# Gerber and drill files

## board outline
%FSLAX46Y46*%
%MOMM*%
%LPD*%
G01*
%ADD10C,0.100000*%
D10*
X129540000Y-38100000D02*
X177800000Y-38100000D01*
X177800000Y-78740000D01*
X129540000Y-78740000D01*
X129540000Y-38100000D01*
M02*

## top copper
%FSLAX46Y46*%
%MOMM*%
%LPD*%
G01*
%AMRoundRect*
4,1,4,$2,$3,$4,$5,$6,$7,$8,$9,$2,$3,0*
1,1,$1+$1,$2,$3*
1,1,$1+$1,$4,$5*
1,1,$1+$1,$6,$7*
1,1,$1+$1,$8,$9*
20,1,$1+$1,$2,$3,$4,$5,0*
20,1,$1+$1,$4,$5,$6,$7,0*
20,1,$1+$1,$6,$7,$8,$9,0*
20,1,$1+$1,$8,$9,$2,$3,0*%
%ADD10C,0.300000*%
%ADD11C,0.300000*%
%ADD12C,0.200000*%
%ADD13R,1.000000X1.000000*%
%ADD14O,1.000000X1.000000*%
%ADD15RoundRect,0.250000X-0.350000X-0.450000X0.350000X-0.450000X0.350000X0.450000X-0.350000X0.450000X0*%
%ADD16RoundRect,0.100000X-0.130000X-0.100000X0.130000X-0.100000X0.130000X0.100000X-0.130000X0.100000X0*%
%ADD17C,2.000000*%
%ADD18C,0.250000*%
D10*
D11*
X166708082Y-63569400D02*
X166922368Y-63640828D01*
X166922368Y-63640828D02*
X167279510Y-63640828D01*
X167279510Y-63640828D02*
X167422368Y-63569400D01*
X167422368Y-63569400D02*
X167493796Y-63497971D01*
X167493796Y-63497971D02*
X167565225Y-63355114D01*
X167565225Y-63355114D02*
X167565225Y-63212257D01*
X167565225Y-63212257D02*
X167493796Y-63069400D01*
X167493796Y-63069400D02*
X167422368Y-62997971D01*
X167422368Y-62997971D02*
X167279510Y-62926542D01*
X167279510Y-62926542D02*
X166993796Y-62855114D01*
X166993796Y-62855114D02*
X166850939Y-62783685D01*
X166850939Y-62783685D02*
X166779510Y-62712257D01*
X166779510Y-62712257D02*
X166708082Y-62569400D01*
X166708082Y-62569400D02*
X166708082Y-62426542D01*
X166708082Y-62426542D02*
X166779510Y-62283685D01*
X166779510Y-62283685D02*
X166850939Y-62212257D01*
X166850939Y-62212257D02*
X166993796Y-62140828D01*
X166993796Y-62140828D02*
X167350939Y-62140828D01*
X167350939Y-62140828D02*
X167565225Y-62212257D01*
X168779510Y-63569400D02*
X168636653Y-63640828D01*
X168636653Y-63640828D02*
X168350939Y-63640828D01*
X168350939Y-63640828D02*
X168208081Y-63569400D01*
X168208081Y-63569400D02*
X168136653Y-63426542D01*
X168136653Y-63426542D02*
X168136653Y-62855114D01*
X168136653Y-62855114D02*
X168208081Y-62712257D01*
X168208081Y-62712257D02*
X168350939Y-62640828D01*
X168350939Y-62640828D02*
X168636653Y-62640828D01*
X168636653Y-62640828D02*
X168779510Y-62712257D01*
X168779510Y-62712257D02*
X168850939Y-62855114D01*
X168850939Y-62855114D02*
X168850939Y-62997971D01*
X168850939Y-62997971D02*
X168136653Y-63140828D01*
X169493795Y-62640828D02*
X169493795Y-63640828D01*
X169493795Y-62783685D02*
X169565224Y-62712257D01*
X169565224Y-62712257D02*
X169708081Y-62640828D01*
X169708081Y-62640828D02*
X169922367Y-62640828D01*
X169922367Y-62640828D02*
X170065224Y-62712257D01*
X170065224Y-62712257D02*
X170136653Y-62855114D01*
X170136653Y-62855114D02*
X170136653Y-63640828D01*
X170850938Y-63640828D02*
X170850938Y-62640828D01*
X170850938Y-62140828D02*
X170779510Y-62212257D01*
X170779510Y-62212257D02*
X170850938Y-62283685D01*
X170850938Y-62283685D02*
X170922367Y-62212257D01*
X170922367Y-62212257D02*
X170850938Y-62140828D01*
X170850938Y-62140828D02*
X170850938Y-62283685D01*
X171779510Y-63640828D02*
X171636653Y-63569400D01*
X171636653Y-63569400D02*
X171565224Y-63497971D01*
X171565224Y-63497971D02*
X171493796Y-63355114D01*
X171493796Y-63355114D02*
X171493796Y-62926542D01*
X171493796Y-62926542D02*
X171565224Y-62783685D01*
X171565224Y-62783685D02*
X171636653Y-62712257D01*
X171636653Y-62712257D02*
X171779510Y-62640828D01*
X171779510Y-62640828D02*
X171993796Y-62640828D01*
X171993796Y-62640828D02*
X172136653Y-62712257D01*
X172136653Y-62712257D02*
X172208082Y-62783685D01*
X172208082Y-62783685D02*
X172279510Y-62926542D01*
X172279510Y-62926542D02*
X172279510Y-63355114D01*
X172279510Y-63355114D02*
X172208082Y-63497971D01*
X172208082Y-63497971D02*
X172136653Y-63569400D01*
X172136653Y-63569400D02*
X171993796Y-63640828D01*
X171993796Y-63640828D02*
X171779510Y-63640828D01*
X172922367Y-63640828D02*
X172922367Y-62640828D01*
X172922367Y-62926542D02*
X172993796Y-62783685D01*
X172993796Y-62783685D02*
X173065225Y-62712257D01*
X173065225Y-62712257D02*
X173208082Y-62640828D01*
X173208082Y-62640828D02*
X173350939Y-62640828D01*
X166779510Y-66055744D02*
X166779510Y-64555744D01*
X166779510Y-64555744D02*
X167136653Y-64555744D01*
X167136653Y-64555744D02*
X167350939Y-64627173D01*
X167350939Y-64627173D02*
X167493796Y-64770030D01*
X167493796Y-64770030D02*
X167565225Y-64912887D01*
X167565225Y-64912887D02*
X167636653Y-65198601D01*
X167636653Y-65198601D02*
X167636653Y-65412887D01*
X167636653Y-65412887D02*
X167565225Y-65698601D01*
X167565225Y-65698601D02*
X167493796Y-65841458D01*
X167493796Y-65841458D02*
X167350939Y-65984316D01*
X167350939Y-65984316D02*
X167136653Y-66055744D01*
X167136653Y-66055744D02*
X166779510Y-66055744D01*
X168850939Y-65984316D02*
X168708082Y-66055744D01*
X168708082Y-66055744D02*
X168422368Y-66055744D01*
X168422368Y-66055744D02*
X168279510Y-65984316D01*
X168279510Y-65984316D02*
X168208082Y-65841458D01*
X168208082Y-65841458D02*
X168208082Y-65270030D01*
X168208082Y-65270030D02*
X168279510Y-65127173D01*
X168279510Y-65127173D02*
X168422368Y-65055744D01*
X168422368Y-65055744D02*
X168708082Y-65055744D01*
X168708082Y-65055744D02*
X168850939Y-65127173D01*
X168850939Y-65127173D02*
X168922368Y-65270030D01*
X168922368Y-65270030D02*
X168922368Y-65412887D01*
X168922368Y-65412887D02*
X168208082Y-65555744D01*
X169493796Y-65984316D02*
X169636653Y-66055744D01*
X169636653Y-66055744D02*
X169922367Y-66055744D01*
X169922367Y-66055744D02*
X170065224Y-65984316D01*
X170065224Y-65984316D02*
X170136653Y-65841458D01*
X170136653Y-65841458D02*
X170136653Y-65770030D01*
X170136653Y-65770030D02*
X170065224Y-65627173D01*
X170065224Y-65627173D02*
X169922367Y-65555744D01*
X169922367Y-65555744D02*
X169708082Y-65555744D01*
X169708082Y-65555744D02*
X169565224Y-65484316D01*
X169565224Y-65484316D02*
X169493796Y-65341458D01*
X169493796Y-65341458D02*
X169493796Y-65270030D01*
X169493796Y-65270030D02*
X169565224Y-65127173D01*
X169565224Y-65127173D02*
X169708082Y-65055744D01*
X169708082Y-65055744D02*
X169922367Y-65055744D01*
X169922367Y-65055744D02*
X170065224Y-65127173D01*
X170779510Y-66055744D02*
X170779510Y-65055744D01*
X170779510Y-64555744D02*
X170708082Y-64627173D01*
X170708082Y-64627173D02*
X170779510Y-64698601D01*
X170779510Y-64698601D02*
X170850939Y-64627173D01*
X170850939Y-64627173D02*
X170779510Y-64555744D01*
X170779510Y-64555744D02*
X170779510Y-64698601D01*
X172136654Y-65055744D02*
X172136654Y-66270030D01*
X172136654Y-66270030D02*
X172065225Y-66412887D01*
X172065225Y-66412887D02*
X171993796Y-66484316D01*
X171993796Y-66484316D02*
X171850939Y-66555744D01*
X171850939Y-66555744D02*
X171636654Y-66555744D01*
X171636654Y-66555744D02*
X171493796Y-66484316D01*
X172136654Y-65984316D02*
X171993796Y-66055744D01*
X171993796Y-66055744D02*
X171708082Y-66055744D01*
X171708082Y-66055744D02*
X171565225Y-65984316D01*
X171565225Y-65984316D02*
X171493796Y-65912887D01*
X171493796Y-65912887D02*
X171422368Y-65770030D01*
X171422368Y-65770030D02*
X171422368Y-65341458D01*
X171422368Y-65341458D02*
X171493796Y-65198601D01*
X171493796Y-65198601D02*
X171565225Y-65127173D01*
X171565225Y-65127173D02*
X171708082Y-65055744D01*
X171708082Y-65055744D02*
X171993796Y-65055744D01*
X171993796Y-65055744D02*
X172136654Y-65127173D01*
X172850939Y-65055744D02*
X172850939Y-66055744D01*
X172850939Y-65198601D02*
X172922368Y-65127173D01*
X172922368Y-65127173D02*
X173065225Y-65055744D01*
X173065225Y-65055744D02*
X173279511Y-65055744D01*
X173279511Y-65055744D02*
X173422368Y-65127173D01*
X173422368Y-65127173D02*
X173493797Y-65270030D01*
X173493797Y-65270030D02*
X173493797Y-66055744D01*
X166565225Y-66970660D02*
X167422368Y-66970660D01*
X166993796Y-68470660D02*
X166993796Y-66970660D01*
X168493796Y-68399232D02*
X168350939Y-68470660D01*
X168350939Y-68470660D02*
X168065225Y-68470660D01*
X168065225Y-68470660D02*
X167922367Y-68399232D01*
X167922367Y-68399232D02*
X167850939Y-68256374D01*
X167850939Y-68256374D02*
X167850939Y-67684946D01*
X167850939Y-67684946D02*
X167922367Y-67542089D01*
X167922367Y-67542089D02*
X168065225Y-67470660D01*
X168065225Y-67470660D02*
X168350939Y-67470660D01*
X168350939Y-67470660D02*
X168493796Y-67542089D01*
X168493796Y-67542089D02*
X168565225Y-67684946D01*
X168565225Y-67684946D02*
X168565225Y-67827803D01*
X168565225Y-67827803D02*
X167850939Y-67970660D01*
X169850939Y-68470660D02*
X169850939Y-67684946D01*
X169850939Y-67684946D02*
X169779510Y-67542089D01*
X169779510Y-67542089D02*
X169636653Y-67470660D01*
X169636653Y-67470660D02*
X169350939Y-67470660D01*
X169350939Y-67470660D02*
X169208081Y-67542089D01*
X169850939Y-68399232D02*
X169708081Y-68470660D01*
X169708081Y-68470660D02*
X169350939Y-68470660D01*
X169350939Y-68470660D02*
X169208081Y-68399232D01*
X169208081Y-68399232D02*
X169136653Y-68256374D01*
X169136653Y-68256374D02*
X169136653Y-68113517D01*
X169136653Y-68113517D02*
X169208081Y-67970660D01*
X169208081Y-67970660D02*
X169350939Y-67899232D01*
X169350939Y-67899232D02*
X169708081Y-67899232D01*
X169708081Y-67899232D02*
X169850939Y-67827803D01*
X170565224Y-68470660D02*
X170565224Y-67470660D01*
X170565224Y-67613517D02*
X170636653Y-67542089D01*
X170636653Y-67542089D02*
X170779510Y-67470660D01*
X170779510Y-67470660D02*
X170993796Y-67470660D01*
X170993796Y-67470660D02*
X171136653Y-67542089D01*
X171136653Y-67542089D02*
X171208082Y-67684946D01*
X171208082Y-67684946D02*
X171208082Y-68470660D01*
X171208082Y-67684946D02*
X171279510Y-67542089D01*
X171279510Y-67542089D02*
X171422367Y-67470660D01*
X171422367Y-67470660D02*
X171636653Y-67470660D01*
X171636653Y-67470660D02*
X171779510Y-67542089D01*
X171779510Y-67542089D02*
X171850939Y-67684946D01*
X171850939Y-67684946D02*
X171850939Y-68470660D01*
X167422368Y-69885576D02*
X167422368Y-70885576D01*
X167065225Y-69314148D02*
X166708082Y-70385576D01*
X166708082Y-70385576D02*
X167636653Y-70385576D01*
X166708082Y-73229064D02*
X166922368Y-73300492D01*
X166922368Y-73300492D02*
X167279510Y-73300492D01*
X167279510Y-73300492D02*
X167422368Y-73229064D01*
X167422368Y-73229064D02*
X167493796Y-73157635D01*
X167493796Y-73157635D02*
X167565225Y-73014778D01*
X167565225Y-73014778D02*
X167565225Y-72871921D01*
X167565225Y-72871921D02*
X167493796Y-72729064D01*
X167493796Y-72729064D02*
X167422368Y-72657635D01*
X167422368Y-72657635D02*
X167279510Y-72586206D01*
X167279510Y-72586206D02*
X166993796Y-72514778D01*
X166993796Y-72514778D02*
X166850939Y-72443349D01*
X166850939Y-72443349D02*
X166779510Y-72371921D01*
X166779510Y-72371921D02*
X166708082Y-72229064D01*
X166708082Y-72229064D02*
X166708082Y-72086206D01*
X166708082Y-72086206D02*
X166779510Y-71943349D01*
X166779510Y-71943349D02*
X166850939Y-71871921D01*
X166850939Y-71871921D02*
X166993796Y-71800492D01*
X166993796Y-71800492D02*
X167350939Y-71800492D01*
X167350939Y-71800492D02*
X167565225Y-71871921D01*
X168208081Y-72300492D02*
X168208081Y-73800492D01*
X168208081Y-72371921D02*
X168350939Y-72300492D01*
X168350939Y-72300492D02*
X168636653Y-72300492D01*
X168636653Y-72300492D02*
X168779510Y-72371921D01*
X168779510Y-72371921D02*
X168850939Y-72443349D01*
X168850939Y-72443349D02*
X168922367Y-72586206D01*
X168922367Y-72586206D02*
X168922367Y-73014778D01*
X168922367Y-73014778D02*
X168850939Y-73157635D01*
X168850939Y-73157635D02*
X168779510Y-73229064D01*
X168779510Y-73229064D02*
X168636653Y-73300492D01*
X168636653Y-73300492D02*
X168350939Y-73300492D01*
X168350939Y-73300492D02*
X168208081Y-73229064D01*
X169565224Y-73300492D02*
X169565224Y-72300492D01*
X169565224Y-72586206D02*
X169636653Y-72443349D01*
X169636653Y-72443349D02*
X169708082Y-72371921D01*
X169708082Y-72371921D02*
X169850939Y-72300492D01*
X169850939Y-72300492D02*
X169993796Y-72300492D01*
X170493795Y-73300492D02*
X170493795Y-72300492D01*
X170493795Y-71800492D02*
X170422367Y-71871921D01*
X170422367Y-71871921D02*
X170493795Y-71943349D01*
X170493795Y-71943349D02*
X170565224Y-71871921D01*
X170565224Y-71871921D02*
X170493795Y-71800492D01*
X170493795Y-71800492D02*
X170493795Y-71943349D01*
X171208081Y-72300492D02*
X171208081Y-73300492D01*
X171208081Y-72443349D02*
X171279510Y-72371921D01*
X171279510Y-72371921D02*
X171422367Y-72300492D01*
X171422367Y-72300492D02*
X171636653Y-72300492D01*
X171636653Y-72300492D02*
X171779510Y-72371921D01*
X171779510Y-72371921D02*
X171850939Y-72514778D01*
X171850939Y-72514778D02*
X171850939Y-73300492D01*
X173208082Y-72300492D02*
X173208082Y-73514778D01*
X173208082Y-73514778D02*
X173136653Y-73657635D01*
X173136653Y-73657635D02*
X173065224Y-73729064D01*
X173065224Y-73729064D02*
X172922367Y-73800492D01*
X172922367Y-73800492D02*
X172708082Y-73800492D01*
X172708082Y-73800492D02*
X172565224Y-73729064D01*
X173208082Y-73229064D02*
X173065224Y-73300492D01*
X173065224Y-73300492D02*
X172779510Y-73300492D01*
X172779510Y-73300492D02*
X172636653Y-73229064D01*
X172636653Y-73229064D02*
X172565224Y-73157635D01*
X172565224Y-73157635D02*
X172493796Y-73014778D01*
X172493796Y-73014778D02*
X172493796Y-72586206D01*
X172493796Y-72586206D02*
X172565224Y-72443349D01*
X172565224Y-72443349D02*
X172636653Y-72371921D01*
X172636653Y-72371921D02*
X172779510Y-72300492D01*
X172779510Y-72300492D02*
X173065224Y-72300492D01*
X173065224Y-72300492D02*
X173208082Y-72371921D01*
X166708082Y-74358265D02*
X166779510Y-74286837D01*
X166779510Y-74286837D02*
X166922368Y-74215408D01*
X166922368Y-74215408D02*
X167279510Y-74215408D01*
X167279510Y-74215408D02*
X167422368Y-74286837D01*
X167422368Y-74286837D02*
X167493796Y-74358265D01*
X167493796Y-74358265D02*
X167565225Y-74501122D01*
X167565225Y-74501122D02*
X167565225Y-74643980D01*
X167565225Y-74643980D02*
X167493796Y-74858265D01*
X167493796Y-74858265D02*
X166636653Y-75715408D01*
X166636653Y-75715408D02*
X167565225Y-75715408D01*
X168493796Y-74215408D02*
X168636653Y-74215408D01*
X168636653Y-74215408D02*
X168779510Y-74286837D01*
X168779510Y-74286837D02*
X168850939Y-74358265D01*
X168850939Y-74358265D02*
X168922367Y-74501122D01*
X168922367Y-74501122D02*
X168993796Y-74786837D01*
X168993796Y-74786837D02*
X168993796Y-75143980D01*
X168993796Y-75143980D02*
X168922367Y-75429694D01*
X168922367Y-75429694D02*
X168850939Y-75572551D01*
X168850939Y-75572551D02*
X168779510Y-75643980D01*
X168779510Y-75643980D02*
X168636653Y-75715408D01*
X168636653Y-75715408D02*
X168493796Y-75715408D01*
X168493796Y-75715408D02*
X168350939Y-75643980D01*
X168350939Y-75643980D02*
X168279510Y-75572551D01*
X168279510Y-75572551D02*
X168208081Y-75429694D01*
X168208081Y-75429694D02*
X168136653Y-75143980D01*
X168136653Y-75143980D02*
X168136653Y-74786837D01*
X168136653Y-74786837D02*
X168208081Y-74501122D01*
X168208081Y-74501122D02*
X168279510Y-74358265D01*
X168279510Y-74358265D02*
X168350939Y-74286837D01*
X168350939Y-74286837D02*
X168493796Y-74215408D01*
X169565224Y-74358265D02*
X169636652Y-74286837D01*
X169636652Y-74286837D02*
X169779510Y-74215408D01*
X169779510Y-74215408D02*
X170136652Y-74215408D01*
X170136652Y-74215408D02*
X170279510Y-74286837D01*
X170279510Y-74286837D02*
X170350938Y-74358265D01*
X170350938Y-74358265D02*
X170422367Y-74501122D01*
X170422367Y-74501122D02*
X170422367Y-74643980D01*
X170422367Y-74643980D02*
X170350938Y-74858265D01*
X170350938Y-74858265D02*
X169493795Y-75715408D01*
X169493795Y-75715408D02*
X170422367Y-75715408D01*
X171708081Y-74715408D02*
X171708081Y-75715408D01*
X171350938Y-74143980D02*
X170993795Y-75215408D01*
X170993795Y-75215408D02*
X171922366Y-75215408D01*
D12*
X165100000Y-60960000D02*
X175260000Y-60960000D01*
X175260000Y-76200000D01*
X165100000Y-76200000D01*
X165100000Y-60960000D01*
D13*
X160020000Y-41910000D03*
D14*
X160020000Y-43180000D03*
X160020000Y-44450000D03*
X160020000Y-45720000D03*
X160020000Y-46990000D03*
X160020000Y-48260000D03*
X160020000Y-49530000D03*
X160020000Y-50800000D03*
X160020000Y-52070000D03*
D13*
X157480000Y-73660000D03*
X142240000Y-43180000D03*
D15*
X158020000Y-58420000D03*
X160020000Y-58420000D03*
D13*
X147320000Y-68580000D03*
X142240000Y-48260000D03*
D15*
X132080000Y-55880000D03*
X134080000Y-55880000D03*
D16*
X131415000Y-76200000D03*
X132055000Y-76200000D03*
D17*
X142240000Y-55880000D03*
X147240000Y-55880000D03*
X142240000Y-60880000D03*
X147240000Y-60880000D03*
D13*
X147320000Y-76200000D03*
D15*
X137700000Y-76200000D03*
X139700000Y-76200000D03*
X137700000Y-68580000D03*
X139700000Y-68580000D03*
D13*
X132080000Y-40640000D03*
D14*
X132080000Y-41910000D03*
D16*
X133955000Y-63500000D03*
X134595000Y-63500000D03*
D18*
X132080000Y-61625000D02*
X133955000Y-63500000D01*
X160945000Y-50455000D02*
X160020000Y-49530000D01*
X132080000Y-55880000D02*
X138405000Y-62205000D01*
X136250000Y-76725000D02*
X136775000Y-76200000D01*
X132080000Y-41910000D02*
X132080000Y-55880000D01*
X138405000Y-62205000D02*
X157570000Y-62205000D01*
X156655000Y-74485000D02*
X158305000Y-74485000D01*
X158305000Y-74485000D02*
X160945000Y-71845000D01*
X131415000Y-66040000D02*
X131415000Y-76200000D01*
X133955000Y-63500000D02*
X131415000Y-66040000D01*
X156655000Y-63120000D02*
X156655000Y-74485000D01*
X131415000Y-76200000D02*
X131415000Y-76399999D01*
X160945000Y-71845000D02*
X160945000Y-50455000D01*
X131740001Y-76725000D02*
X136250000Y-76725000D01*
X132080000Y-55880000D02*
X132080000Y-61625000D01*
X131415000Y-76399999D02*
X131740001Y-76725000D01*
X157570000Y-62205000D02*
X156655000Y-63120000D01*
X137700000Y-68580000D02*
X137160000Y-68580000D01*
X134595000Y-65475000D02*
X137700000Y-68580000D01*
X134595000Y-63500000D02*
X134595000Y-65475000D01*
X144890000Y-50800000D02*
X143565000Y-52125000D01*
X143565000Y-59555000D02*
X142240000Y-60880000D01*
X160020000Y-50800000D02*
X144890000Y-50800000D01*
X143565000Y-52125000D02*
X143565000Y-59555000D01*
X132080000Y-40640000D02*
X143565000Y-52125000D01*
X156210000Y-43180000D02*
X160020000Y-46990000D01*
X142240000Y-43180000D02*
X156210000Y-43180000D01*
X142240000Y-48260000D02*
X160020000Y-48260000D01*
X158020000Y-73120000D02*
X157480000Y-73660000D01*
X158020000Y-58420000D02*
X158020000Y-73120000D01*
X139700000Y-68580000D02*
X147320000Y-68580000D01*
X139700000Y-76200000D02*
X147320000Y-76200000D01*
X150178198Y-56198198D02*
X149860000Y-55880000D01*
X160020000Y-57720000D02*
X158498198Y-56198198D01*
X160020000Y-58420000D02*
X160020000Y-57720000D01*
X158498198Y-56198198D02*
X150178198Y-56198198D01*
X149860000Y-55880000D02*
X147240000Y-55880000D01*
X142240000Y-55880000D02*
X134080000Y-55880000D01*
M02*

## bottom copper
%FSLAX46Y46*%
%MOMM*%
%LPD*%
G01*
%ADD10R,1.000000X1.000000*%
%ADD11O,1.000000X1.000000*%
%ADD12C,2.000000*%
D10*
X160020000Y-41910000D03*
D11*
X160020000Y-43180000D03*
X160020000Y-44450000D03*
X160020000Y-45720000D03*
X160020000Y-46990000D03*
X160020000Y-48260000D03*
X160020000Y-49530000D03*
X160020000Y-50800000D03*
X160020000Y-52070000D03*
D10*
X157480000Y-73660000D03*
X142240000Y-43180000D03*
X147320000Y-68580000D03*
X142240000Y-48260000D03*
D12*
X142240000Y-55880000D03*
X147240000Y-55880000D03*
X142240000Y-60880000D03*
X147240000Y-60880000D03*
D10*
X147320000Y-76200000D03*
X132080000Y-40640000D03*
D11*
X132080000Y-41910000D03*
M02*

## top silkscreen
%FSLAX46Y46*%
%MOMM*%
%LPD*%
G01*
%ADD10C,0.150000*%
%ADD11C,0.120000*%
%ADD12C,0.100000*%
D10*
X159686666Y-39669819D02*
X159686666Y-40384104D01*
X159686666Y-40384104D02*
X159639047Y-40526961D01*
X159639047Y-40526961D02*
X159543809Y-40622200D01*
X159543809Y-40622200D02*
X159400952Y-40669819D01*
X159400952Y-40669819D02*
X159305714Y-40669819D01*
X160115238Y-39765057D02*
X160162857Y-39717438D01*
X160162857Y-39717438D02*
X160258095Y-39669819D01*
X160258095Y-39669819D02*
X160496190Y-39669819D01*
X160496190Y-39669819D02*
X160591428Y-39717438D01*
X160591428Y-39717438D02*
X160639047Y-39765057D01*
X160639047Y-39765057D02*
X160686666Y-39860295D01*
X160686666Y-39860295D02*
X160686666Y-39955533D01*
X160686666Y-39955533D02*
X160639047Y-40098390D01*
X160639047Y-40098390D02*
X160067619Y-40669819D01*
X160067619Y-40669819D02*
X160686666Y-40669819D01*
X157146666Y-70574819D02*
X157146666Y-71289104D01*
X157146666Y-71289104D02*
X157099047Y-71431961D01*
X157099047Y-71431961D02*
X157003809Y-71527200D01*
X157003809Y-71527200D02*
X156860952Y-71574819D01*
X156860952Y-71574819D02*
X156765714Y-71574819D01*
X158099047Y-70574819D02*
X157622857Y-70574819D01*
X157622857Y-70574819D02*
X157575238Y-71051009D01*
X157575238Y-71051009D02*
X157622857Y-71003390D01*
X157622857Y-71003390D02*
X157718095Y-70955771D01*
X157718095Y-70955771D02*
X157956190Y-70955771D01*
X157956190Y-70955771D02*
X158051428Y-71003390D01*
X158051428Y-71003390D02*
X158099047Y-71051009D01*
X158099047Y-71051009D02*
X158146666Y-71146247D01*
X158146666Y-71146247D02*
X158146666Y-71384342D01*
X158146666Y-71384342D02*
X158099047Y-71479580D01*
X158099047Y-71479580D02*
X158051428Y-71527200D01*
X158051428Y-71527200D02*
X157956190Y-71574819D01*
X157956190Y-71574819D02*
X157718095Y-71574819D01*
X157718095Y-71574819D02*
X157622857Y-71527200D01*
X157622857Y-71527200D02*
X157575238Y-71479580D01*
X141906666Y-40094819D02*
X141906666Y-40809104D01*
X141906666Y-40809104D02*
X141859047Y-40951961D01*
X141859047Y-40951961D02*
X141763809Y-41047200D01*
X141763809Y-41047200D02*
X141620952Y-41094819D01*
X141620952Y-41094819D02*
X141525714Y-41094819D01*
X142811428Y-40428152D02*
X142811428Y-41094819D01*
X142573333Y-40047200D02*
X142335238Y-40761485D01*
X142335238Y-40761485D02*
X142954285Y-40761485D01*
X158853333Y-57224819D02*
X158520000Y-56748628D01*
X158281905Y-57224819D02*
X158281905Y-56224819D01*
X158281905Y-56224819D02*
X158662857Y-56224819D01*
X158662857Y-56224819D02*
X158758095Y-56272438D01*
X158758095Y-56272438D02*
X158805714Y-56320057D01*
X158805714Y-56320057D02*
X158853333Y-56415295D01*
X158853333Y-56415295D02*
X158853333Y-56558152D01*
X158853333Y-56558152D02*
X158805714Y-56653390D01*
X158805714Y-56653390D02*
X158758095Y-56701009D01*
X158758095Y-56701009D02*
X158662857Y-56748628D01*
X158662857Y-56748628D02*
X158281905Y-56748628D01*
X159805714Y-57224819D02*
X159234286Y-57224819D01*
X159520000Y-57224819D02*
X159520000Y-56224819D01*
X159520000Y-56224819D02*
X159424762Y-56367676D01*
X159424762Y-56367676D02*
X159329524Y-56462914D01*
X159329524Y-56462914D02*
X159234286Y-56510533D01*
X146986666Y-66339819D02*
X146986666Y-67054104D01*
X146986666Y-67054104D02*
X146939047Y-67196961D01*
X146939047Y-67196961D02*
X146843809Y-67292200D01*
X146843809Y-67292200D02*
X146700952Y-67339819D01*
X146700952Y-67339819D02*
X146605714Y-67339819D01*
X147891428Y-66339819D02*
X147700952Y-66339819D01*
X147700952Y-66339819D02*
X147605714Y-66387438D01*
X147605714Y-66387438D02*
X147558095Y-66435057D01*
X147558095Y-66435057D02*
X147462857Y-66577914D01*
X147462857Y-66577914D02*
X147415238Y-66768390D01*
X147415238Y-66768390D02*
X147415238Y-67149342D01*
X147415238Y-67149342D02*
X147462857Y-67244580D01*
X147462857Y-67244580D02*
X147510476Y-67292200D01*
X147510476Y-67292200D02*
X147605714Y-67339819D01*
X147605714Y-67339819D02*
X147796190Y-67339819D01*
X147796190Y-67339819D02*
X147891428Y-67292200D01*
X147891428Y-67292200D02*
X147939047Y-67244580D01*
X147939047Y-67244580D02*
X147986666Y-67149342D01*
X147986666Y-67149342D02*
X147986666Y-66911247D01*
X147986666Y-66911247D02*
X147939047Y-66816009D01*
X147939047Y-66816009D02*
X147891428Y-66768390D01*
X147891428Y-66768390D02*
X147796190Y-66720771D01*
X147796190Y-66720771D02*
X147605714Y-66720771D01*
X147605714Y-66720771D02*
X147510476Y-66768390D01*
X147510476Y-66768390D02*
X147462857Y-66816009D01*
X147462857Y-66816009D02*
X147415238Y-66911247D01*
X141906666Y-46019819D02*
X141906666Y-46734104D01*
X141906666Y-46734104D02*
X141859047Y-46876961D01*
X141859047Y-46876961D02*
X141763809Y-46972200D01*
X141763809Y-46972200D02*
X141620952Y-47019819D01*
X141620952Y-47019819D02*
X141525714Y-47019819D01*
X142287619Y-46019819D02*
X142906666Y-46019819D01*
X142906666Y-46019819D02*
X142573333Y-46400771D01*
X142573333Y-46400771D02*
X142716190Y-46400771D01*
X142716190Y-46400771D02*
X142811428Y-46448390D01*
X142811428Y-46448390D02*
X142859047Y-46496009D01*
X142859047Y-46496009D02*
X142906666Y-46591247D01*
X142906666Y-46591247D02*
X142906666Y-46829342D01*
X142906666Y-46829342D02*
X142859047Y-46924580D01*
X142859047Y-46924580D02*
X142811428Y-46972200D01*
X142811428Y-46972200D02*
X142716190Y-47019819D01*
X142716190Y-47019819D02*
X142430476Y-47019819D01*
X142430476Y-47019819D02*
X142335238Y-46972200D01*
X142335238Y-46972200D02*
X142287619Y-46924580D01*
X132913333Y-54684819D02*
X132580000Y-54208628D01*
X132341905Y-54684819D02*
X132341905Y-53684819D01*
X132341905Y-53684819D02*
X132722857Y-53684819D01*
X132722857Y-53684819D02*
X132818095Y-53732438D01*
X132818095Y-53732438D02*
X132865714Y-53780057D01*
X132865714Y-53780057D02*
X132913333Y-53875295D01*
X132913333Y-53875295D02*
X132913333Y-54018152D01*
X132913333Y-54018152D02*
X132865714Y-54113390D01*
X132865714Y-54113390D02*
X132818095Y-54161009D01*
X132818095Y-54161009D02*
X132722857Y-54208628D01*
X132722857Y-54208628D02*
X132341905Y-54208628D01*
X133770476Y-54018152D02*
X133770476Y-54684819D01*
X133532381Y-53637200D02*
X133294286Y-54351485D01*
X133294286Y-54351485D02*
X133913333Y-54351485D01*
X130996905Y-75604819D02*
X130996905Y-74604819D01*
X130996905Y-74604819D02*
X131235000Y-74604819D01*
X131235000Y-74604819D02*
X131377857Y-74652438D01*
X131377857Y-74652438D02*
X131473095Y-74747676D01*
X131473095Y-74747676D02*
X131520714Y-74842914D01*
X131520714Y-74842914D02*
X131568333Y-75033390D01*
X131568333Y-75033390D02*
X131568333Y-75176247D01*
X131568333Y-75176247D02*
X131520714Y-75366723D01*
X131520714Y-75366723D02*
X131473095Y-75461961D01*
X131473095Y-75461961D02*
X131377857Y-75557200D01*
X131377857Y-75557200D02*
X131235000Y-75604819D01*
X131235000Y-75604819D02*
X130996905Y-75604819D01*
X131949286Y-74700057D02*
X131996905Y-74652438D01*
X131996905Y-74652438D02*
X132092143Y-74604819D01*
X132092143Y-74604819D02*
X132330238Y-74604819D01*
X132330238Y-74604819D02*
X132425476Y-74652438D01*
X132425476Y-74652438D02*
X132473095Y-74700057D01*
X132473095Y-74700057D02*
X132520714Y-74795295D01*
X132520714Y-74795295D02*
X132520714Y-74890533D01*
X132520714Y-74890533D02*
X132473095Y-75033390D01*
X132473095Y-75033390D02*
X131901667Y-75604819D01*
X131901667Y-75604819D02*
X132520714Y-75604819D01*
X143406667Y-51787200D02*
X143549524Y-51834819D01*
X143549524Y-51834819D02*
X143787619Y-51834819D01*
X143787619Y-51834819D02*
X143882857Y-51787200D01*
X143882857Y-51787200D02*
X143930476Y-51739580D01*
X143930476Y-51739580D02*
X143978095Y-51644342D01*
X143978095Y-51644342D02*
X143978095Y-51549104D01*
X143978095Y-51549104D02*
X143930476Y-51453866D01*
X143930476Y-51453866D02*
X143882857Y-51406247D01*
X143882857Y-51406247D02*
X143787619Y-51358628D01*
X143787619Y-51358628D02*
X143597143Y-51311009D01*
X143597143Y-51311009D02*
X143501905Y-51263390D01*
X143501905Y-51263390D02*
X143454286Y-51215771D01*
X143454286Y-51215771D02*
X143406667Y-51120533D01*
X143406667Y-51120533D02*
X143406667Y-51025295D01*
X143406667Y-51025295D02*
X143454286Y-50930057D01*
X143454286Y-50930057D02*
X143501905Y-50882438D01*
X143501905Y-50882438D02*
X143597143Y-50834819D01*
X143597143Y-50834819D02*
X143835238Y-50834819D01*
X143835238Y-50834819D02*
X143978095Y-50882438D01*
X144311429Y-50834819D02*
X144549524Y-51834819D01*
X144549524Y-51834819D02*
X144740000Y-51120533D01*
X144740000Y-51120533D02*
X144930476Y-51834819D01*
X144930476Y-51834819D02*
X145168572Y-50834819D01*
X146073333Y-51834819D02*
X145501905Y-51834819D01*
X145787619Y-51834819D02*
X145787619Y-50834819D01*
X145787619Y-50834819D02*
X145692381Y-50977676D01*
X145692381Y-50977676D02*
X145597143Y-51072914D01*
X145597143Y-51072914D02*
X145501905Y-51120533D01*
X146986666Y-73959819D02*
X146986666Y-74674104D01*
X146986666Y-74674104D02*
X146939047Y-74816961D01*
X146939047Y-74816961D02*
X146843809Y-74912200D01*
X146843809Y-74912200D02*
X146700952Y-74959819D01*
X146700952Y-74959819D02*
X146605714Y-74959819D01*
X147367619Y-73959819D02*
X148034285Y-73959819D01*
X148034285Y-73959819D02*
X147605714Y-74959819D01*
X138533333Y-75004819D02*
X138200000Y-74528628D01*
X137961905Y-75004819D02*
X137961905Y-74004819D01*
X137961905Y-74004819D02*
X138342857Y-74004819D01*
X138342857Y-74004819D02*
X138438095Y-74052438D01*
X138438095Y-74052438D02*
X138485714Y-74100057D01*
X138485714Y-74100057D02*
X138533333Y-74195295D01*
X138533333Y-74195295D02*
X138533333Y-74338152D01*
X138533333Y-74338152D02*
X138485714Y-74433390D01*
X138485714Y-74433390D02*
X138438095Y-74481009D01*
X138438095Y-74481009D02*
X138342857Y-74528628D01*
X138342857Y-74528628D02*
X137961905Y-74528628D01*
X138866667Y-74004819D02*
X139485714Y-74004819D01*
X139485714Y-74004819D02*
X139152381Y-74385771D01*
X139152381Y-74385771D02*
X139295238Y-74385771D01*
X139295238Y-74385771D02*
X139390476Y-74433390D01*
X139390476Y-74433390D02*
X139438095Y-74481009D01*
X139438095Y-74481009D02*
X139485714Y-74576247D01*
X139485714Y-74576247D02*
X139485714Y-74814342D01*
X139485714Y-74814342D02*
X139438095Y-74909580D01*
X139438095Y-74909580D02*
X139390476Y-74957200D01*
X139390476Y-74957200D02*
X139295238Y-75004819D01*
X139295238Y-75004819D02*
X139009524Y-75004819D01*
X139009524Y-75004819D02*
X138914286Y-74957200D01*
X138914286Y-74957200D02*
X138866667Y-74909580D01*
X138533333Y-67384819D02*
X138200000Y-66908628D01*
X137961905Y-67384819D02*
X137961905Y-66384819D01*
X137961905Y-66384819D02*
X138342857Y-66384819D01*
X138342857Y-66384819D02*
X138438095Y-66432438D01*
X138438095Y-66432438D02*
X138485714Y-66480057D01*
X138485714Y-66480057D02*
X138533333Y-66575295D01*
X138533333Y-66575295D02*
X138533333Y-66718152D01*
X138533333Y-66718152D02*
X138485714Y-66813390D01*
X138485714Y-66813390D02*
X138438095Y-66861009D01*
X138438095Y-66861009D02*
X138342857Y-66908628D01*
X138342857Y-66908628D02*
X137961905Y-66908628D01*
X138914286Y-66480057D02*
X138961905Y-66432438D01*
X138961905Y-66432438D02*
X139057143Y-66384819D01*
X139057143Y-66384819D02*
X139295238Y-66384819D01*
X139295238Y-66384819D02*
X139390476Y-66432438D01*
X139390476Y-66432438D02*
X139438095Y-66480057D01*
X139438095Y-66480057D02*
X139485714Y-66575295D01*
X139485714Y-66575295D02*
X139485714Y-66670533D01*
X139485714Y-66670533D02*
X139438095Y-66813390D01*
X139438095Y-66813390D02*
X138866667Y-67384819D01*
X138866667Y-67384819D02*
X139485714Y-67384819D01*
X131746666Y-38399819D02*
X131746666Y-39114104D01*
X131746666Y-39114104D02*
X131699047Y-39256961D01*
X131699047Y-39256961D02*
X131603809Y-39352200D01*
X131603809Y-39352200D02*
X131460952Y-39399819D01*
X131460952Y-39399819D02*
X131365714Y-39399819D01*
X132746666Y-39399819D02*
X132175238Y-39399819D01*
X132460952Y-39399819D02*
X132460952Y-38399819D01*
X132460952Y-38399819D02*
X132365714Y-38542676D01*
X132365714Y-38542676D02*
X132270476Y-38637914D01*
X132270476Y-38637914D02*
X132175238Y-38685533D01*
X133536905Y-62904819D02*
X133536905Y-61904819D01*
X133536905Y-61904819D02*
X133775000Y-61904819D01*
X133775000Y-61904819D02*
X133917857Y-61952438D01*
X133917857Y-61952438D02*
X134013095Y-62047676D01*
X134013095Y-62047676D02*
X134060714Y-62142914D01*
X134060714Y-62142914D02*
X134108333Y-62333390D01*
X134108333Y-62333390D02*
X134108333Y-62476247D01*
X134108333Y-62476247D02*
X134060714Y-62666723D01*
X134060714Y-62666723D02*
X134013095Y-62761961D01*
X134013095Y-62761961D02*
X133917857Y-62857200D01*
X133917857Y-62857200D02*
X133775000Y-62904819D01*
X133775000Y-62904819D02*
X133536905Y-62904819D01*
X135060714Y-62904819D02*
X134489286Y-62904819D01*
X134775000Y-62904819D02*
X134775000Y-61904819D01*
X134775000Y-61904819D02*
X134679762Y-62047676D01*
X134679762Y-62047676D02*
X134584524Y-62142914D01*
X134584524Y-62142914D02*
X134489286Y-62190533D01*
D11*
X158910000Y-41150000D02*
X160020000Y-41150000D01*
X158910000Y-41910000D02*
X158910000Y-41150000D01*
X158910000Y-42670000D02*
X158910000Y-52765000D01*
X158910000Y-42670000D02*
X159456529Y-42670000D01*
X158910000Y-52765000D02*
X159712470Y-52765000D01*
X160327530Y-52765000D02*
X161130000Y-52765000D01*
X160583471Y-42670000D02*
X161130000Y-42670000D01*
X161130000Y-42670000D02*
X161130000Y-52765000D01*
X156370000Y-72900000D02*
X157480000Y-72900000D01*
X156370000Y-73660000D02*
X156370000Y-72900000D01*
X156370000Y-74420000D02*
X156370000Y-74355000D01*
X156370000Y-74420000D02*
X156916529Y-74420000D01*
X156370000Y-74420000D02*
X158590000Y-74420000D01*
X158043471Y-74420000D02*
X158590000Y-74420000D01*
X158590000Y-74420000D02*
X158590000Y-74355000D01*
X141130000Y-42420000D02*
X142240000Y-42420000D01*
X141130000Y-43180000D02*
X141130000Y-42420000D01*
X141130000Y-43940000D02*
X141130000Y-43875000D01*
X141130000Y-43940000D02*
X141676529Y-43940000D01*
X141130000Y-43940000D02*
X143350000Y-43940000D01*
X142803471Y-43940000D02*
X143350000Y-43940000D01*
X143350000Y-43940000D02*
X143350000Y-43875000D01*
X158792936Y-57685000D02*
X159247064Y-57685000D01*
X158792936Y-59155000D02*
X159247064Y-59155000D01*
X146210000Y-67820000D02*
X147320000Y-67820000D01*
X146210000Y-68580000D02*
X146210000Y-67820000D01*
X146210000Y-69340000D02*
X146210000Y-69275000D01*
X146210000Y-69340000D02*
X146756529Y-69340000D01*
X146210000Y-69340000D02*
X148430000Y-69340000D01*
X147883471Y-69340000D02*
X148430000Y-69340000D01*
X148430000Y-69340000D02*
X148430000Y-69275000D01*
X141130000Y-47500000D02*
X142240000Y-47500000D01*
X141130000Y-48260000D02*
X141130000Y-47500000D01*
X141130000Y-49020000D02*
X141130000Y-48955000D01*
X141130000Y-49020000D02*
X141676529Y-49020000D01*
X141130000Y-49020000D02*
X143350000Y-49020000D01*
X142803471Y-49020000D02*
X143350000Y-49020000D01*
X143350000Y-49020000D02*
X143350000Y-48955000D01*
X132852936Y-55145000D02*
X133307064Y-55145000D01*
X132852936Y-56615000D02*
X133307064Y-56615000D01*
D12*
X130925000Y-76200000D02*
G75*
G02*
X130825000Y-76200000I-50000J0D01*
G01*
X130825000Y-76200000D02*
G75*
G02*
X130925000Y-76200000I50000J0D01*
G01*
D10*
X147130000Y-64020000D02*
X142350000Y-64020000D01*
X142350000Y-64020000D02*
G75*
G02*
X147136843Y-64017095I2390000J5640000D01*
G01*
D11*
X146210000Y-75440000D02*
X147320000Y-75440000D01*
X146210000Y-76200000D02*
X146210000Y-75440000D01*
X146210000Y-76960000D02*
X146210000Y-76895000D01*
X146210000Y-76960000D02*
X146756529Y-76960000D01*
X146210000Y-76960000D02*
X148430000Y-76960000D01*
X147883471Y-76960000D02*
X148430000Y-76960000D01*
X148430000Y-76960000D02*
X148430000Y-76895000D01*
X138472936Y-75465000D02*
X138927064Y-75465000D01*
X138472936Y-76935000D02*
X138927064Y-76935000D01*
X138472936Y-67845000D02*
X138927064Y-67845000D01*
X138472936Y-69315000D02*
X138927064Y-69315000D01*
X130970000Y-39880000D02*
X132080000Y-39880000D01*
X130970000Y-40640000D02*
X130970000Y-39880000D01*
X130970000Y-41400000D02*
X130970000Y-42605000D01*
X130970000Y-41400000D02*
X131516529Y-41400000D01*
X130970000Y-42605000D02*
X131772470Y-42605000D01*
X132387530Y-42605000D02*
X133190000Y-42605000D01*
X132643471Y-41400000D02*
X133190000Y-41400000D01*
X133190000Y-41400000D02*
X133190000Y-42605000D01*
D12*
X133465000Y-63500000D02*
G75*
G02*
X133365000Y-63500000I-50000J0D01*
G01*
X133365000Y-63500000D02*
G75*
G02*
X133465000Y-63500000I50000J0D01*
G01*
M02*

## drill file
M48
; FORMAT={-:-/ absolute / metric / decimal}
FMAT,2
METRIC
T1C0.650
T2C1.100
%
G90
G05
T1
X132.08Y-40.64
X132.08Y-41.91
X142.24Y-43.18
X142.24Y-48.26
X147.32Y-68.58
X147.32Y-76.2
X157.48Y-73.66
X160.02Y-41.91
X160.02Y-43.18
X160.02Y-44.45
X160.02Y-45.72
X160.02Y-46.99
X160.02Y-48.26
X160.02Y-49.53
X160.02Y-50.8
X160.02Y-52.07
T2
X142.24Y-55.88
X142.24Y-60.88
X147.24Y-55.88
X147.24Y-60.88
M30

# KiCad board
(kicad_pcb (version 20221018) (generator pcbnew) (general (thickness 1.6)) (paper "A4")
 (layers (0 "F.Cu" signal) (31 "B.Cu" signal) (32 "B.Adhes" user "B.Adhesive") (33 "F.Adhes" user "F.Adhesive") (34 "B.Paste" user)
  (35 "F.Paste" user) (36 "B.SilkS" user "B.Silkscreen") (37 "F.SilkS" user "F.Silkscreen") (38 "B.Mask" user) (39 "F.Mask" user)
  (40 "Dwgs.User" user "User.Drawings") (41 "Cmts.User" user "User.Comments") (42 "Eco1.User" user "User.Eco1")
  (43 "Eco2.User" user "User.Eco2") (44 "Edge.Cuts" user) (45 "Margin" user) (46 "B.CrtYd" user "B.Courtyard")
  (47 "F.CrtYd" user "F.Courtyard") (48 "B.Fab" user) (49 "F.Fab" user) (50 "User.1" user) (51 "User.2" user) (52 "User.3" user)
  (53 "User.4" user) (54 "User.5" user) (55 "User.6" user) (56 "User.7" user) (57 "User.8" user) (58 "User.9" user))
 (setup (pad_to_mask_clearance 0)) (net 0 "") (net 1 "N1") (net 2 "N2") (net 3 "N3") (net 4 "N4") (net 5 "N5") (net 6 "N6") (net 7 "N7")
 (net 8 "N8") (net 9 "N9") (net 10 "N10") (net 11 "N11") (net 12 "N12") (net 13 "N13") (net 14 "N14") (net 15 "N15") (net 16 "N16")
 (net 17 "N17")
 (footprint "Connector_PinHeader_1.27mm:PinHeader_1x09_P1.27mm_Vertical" (layer "F.Cu") (at 160.02 41.91)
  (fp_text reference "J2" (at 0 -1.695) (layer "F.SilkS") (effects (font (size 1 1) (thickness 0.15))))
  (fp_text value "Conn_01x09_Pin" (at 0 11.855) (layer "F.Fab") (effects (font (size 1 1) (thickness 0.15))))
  (fp_line (start -1.11 -0.76) (end 0 -0.76) (stroke (width 0.12) (type solid)) (layer "F.SilkS"))
  (fp_line (start -1.11 0) (end -1.11 -0.76) (stroke (width 0.12) (type solid)) (layer "F.SilkS"))
  (fp_line (start -1.11 0.76) (end -1.11 10.855) (stroke (width 0.12) (type solid)) (layer "F.SilkS"))
  (fp_line (start -1.11 0.76) (end -0.563471 0.76) (stroke (width 0.12) (type solid)) (layer "F.SilkS"))
  (fp_line (start -1.11 10.855) (end -0.30753 10.855) (stroke (width 0.12) (type solid)) (layer "F.SilkS"))
  (fp_line (start 0.30753 10.855) (end 1.11 10.855) (stroke (width 0.12) (type solid)) (layer "F.SilkS"))
  (fp_line (start 0.563471 0.76) (end 1.11 0.76) (stroke (width 0.12) (type solid)) (layer "F.SilkS"))
  (fp_line (start 1.11 0.76) (end 1.11 10.855) (stroke (width 0.12) (type solid)) (layer "F.SilkS"))
  (pad "1" thru_hole rect (at 0 0) (size 1 1) (drill 0.65) (layers "*.Cu" "*.Mask") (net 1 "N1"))
  (pad "2" thru_hole oval (at 0 1.27) (size 1 1) (drill 0.65) (layers "*.Cu" "*.Mask") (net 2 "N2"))
  (pad "3" thru_hole oval (at 0 2.54) (size 1 1) (drill 0.65) (layers "*.Cu" "*.Mask") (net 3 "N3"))
  (pad "4" thru_hole oval (at 0 3.81) (size 1 1) (drill 0.65) (layers "*.Cu" "*.Mask") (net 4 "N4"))
  (pad "5" thru_hole oval (at 0 5.08) (size 1 1) (drill 0.65) (layers "*.Cu" "*.Mask") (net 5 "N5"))
  (pad "6" thru_hole oval (at 0 6.35) (size 1 1) (drill 0.65) (layers "*.Cu" "*.Mask") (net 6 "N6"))
  (pad "7" thru_hole oval (at 0 7.62) (size 1 1) (drill 0.65) (layers "*.Cu" "*.Mask") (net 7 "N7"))
  (pad "8" thru_hole oval (at 0 8.89) (size 1 1) (drill 0.65) (layers "*.Cu" "*.Mask") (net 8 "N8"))
  (pad "9" thru_hole oval (at 0 10.16) (size 1 1) (drill 0.65) (layers "*.Cu" "*.Mask") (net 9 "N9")))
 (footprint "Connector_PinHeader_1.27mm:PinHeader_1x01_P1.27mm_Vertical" (layer "F.Cu") (at 157.48 73.66)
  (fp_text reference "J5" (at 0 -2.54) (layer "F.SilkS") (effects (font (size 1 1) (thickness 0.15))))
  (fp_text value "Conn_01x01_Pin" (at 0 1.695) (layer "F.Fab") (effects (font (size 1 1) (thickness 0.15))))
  (fp_line (start -1.11 -0.76) (end 0 -0.76) (stroke (width 0.12) (type solid)) (layer "F.SilkS"))
  (fp_line (start -1.11 0) (end -1.11 -0.76) (stroke (width 0.12) (type solid)) (layer "F.SilkS"))
  (fp_line (start -1.11 0.76) (end -1.11 0.695) (stroke (width 0.12) (type solid)) (layer "F.SilkS"))
  (fp_line (start -1.11 0.76) (end -0.563471 0.76) (stroke (width 0.12) (type solid)) (layer "F.SilkS"))
  (fp_line (start -1.11 0.76) (end 1.11 0.76) (stroke (width 0.12) (type solid)) (layer "F.SilkS"))
  (fp_line (start 0.563471 0.76) (end 1.11 0.76) (stroke (width 0.12) (type solid)) (layer "F.SilkS"))
  (fp_line (start 1.11 0.76) (end 1.11 0.695) (stroke (width 0.12) (type solid)) (layer "F.SilkS"))
  (pad "1" thru_hole rect (at 0 0) (size 1 1) (drill 0.65) (layers "*.Cu" "*.Mask") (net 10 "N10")))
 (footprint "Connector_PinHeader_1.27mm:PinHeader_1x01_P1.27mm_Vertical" (layer "F.Cu") (at 142.24 43.18)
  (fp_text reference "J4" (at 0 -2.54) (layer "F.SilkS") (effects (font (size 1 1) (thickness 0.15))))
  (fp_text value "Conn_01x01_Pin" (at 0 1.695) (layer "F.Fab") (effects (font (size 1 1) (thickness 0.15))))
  (fp_line (start -1.11 -0.76) (end 0 -0.76) (stroke (width 0.12) (type solid)) (layer "F.SilkS"))
  (fp_line (start -1.11 0) (end -1.11 -0.76) (stroke (width 0.12) (type solid)) (layer "F.SilkS"))
  (fp_line (start -1.11 0.76) (end -1.11 0.695) (stroke (width 0.12) (type solid)) (layer "F.SilkS"))
  (fp_line (start -1.11 0.76) (end -0.563471 0.76) (stroke (width 0.12) (type solid)) (layer "F.SilkS"))
  (fp_line (start -1.11 0.76) (end 1.11 0.76) (stroke (width 0.12) (type solid)) (layer "F.SilkS"))
  (fp_line (start 0.563471 0.76) (end 1.11 0.76) (stroke (width 0.12) (type solid)) (layer "F.SilkS"))
  (fp_line (start 1.11 0.76) (end 1.11 0.695) (stroke (width 0.12) (type solid)) (layer "F.SilkS"))
  (pad "1" thru_hole rect (at 0 0) (size 1 1) (drill 0.65) (layers "*.Cu" "*.Mask") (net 5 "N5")))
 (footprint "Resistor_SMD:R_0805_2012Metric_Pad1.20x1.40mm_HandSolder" (layer "F.Cu") (at 159.02 58.42)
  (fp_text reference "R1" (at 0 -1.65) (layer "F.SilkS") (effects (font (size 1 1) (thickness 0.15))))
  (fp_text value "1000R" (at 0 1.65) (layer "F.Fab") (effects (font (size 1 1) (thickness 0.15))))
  (fp_line (start -0.227064 -0.735) (end 0.227064 -0.735) (stroke (width 0.12) (type solid)) (layer "F.SilkS"))
  (fp_line (start -0.227064 0.735) (end 0.227064 0.735) (stroke (width 0.12) (type solid)) (layer "F.SilkS"))
  (pad "1" smd roundrect (at -1 0) (size 1.2 1.4) (layers "F.Cu" "F.Paste" "F.Mask") (roundrect_rratio 0.2083333333) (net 10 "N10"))
  (pad "2" smd roundrect (at 1 0) (size 1.2 1.4) (layers "F.Cu" "F.Paste" "F.Mask") (roundrect_rratio 0.2083333333) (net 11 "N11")))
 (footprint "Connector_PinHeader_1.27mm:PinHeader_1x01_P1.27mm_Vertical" (layer "F.Cu") (at 147.32 68.58)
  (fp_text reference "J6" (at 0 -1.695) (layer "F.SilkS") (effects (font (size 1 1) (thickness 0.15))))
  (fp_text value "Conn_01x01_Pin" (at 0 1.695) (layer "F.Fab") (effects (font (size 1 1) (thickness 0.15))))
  (fp_line (start -1.11 -0.76) (end 0 -0.76) (stroke (width 0.12) (type solid)) (layer "F.SilkS"))
  (fp_line (start -1.11 0) (end -1.11 -0.76) (stroke (width 0.12) (type solid)) (layer "F.SilkS"))
  (fp_line (start -1.11 0.76) (end -1.11 0.695) (stroke (width 0.12) (type solid)) (layer "F.SilkS"))
  (fp_line (start -1.11 0.76) (end -0.563471 0.76) (stroke (width 0.12) (type solid)) (layer "F.SilkS"))
  (fp_line (start -1.11 0.76) (end 1.11 0.76) (stroke (width 0.12) (type solid)) (layer "F.SilkS"))
  (fp_line (start 0.563471 0.76) (end 1.11 0.76) (stroke (width 0.12) (type solid)) (layer "F.SilkS"))
  (fp_line (start 1.11 0.76) (end 1.11 0.695) (stroke (width 0.12) (type solid)) (layer "F.SilkS"))
  (pad "1" thru_hole rect (at 0 0) (size 1 1) (drill 0.65) (layers "*.Cu" "*.Mask") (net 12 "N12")))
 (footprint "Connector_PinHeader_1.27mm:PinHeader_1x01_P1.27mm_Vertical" (layer "F.Cu") (at 142.24 48.26)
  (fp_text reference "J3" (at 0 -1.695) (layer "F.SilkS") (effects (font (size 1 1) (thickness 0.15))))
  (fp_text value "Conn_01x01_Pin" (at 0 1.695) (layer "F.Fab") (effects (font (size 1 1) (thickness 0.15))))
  (fp_line (start -1.11 -0.76) (end 0 -0.76) (stroke (width 0.12) (type solid)) (layer "F.SilkS"))
  (fp_line (start -1.11 0) (end -1.11 -0.76) (stroke (width 0.12) (type solid)) (layer "F.SilkS"))
  (fp_line (start -1.11 0.76) (end -1.11 0.695) (stroke (width 0.12) (type solid)) (layer "F.SilkS"))
  (fp_line (start -1.11 0.76) (end -0.563471 0.76) (stroke (width 0.12) (type solid)) (layer "F.SilkS"))
  (fp_line (start -1.11 0.76) (end 1.11 0.76) (stroke (width 0.12) (type solid)) (layer "F.SilkS"))
  (fp_line (start 0.563471 0.76) (end 1.11 0.76) (stroke (width 0.12) (type solid)) (layer "F.SilkS"))
  (fp_line (start 1.11 0.76) (end 1.11 0.695) (stroke (width 0.12) (type solid)) (layer "F.SilkS"))
  (pad "1" thru_hole rect (at 0 0) (size 1 1) (drill 0.65) (layers "*.Cu" "*.Mask") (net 6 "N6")))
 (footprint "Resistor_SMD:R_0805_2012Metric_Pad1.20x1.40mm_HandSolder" (layer "F.Cu") (at 133.08 55.88)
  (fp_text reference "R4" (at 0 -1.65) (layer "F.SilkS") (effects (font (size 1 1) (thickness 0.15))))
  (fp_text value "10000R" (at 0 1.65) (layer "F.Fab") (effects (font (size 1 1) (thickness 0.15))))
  (fp_line (start -0.227064 -0.735) (end 0.227064 -0.735) (stroke (width 0.12) (type solid)) (layer "F.SilkS"))
  (fp_line (start -0.227064 0.735) (end 0.227064 0.735) (stroke (width 0.12) (type solid)) (layer "F.SilkS"))
  (pad "1" smd roundrect (at -1 0) (size 1.2 1.4) (layers "F.Cu" "F.Paste" "F.Mask") (roundrect_rratio 0.2083333333) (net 7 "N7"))
  (pad "2" smd roundrect (at 1 0) (size 1.2 1.4) (layers "F.Cu" "F.Paste" "F.Mask") (roundrect_rratio 0.2083333333) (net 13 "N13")))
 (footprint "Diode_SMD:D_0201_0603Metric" (layer "F.Cu") (at 131.735 76.2)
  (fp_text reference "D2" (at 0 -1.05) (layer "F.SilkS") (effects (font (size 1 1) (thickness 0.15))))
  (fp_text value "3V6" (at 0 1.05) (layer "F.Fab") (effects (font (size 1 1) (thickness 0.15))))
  (fp_circle (center -0.86 0) (end -0.81 0) (stroke (width 0.1) (type solid)) (fill none) (layer "F.SilkS"))
  (pad "" smd roundrect (at -0.345 0) (size 0.318 0.36) (layers "F.Paste") (roundrect_rratio 0.25))
  (pad "" smd roundrect (at 0.345 0) (size 0.318 0.36) (layers "F.Paste") (roundrect_rratio 0.25))
  (pad "1" smd roundrect (at -0.32 0) (size 0.46 0.4) (layers "F.Cu" "F.Mask") (roundrect_rratio 0.25) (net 7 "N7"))
  (pad "2" smd roundrect (at 0.32 0) (size 0.46 0.4) (layers "F.Cu" "F.Mask") (roundrect_rratio 0.25) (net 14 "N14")))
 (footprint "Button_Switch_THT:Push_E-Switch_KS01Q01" (layer "F.Cu") (at 142.24 55.88)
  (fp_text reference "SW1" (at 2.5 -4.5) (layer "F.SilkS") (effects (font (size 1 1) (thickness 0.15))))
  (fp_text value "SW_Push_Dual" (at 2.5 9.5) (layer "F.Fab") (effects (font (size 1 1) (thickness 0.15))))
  (fp_line (start 4.89 8.14) (end 0.11 8.14) (stroke (width 0.15) (type solid)) (layer "F.SilkS"))
  (fp_arc (start 0.11 8.14) (mid 2.496283 -3.625495) (end 4.896843 8.137095) (stroke (width 0.15) (type solid)) (layer "F.SilkS"))
  (pad "1" thru_hole circle (at 0 0) (size 2 2) (drill 1.1) (layers "*.Cu" "*.Mask") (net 13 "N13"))
  (pad "2" thru_hole circle (at 5 0) (size 2 2) (drill 1.1) (layers "*.Cu" "*.Mask") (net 11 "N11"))
  (pad "3" thru_hole circle (at 0 5) (size 2 2) (drill 1.1) (layers "*.Cu" "*.Mask") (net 8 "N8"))
  (pad "4" thru_hole circle (at 5 5) (size 2 2) (drill 1.1) (layers "*.Cu" "*.Mask") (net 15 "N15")))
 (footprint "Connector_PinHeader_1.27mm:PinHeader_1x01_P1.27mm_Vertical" (layer "F.Cu") (at 147.32 76.2)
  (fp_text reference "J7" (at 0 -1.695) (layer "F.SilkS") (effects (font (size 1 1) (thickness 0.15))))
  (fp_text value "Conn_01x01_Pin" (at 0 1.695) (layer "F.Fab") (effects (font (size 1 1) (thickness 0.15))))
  (fp_line (start -1.11 -0.76) (end 0 -0.76) (stroke (width 0.12) (type solid)) (layer "F.SilkS"))
  (fp_line (start -1.11 0) (end -1.11 -0.76) (stroke (width 0.12) (type solid)) (layer "F.SilkS"))
  (fp_line (start -1.11 0.76) (end -1.11 0.695) (stroke (width 0.12) (type solid)) (layer "F.SilkS"))
  (fp_line (start -1.11 0.76) (end -0.563471 0.76) (stroke (width 0.12) (type solid)) (layer "F.SilkS"))
  (fp_line (start -1.11 0.76) (end 1.11 0.76) (stroke (width 0.12) (type solid)) (layer "F.SilkS"))
  (fp_line (start 0.563471 0.76) (end 1.11 0.76) (stroke (width 0.12) (type solid)) (layer "F.SilkS"))
  (fp_line (start 1.11 0.76) (end 1.11 0.695) (stroke (width 0.12) (type solid)) (layer "F.SilkS"))
  (pad "1" thru_hole rect (at 0 0) (size 1 1) (drill 0.65) (layers "*.Cu" "*.Mask") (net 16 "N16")))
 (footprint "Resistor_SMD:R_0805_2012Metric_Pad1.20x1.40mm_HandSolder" (layer "F.Cu") (at 138.7 76.2)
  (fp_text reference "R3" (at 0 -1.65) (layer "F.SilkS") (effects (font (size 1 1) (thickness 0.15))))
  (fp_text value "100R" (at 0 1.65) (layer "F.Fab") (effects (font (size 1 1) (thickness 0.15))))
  (fp_line (start -0.227064 -0.735) (end 0.227064 -0.735) (stroke (width 0.12) (type solid)) (layer "F.SilkS"))
  (fp_line (start -0.227064 0.735) (end 0.227064 0.735) (stroke (width 0.12) (type solid)) (layer "F.SilkS"))
  (pad "1" smd roundrect (at -1 0) (size 1.2 1.4) (layers "F.Cu" "F.Paste" "F.Mask") (roundrect_rratio 0.2083333333) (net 14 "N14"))
  (pad "2" smd roundrect (at 1 0) (size 1.2 1.4) (layers "F.Cu" "F.Paste" "F.Mask") (roundrect_rratio 0.2083333333) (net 16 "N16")))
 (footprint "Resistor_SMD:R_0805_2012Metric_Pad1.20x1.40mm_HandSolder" (layer "F.Cu") (at 138.7 68.58)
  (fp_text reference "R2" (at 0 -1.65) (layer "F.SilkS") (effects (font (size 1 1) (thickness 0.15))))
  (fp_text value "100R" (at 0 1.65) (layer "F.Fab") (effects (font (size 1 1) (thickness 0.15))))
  (fp_line (start -0.227064 -0.735) (end 0.227064 -0.735) (stroke (width 0.12) (type solid)) (layer "F.SilkS"))
  (fp_line (start -0.227064 0.735) (end 0.227064 0.735) (stroke (width 0.12) (type solid)) (layer "F.SilkS"))
  (pad "1" smd roundrect (at -1 0) (size 1.2 1.4) (layers "F.Cu" "F.Paste" "F.Mask") (roundrect_rratio 0.2083333333) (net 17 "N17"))
  (pad "2" smd roundrect (at 1 0) (size 1.2 1.4) (layers "F.Cu" "F.Paste" "F.Mask") (roundrect_rratio 0.2083333333) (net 12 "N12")))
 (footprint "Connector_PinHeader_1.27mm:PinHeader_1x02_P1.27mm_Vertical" (layer "F.Cu") (at 132.08 40.64)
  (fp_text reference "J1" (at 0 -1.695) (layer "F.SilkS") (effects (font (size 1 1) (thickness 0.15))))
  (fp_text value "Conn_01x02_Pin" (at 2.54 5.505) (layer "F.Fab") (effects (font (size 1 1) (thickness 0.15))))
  (fp_line (start -1.11 -0.76) (end 0 -0.76) (stroke (width 0.12) (type solid)) (layer "F.SilkS"))
  (fp_line (start -1.11 0) (end -1.11 -0.76) (stroke (width 0.12) (type solid)) (layer "F.SilkS"))
  (fp_line (start -1.11 0.76) (end -1.11 1.965) (stroke (width 0.12) (type solid)) (layer "F.SilkS"))
  (fp_line (start -1.11 0.76) (end -0.563471 0.76) (stroke (width 0.12) (type solid)) (layer "F.SilkS"))
  (fp_line (start -1.11 1.965) (end -0.30753 1.965) (stroke (width 0.12) (type solid)) (layer "F.SilkS"))
  (fp_line (start 0.30753 1.965) (end 1.11 1.965) (stroke (width 0.12) (type solid)) (layer "F.SilkS"))
  (fp_line (start 0.563471 0.76) (end 1.11 0.76) (stroke (width 0.12) (type solid)) (layer "F.SilkS"))
  (fp_line (start 1.11 0.76) (end 1.11 1.965) (stroke (width 0.12) (type solid)) (layer "F.SilkS"))
  (pad "1" thru_hole rect (at 0 0) (size 1 1) (drill 0.65) (layers "*.Cu" "*.Mask") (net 8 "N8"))
  (pad "2" thru_hole oval (at 0 1.27) (size 1 1) (drill 0.65) (layers "*.Cu" "*.Mask") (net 7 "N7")))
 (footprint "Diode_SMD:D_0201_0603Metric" (layer "F.Cu") (at 134.275 63.5)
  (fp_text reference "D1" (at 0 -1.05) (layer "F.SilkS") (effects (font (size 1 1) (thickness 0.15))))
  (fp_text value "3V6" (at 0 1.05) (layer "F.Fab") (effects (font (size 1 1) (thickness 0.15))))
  (fp_circle (center -0.86 0) (end -0.81 0) (stroke (width 0.1) (type solid)) (fill none) (layer "F.SilkS"))
  (pad "" smd roundrect (at -0.345 0) (size 0.318 0.36) (layers "F.Paste") (roundrect_rratio 0.25))
  (pad "" smd roundrect (at 0.345 0) (size 0.318 0.36) (layers "F.Paste") (roundrect_rratio 0.25))
  (pad "1" smd roundrect (at -0.32 0) (size 0.46 0.4) (layers "F.Cu" "F.Mask") (roundrect_rratio 0.25) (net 7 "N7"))
  (pad "2" smd roundrect (at 0.32 0) (size 0.46 0.4) (layers "F.Cu" "F.Mask") (roundrect_rratio 0.25) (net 17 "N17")))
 (gr_rect (start 129.54 38.1) (end 177.8 78.74) (stroke (width 0.1) (type default)) (fill none) (layer "Edge.Cuts"))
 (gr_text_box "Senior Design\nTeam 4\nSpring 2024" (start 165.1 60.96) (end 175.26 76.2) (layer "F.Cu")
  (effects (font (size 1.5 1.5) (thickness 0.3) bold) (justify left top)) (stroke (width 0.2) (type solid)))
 (segment (start 132.08 61.625) (end 133.955 63.5) (width 0.25) (layer "F.Cu") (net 7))
 (segment (start 160.945 50.455) (end 160.02 49.53) (width 0.25) (layer "F.Cu") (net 7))
 (segment (start 132.08 55.88) (end 138.405 62.205) (width 0.25) (layer "F.Cu") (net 7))
 (segment (start 136.25 76.725) (end 136.775 76.2) (width 0.25) (layer "F.Cu") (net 7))
 (segment (start 132.08 41.91) (end 132.08 55.88) (width 0.25) (layer "F.Cu") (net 7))
 (segment (start 138.405 62.205) (end 157.57 62.205) (width 0.25) (layer "F.Cu") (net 7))
 (segment (start 156.655 74.485) (end 158.305 74.485) (width 0.25) (layer "F.Cu") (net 7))
 (segment (start 158.305 74.485) (end 160.945 71.845) (width 0.25) (layer "F.Cu") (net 7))
 (segment (start 131.415 66.04) (end 131.415 76.2) (width 0.25) (layer "F.Cu") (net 7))
 (segment (start 133.955 63.5) (end 131.415 66.04) (width 0.25) (layer "F.Cu") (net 7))
 (segment (start 156.655 63.12) (end 156.655 74.485) (width 0.25) (layer "F.Cu") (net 7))
 (segment (start 131.415 76.2) (end 131.415 76.399999) (width 0.25) (layer "F.Cu") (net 7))
 (segment (start 160.945 71.845) (end 160.945 50.455) (width 0.25) (layer "F.Cu") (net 7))
 (segment (start 131.740001 76.725) (end 136.25 76.725) (width 0.25) (layer "F.Cu") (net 7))
 (segment (start 132.08 55.88) (end 132.08 61.625) (width 0.25) (layer "F.Cu") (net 7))
 (segment (start 131.415 76.399999) (end 131.740001 76.725) (width 0.25) (layer "F.Cu") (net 7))
 (segment (start 157.57 62.205) (end 156.655 63.12) (width 0.25) (layer "F.Cu") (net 7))
 (segment (start 137.7 68.58) (end 137.16 68.58) (width 0.25) (layer "F.Cu") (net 17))
 (segment (start 134.595 65.475) (end 137.7 68.58) (width 0.25) (layer "F.Cu") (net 17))
 (segment (start 134.595 63.5) (end 134.595 65.475) (width 0.25) (layer "F.Cu") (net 17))
 (segment (start 144.89 50.8) (end 143.565 52.125) (width 0.25) (layer "F.Cu") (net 8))
 (segment (start 143.565 59.555) (end 142.24 60.88) (width 0.25) (layer "F.Cu") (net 8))
 (segment (start 160.02 50.8) (end 144.89 50.8) (width 0.25) (layer "F.Cu") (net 8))
 (segment (start 143.565 52.125) (end 143.565 59.555) (width 0.25) (layer "F.Cu") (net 8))
 (segment (start 132.08 40.64) (end 143.565 52.125) (width 0.25) (layer "F.Cu") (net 8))
 (segment (start 156.21 43.18) (end 160.02 46.99) (width 0.25) (layer "F.Cu") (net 5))
 (segment (start 142.24 43.18) (end 156.21 43.18) (width 0.25) (layer "F.Cu") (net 5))
 (segment (start 142.24 48.26) (end 160.02 48.26) (width 0.25) (layer "F.Cu") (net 6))
 (segment (start 158.02 73.12) (end 157.48 73.66) (width 0.25) (layer "F.Cu") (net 10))
 (segment (start 158.02 58.42) (end 158.02 73.12) (width 0.25) (layer "F.Cu") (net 10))
 (segment (start 139.7 68.58) (end 147.32 68.58) (width 0.25) (layer "F.Cu") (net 12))
 (segment (start 139.7 76.2) (end 147.32 76.2) (width 0.25) (layer "F.Cu") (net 16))
 (segment (start 150.178198 56.198198) (end 149.86 55.88) (width 0.25) (layer "F.Cu") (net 11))
 (segment (start 160.02 57.72) (end 158.498198 56.198198) (width 0.25) (layer "F.Cu") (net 11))
 (segment (start 160.02 58.42) (end 160.02 57.72) (width 0.25) (layer "F.Cu") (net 11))
 (segment (start 158.498198 56.198198) (end 150.178198 56.198198) (width 0.25) (layer "F.Cu") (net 11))
 (segment (start 149.86 55.88) (end 147.24 55.88) (width 0.25) (layer "F.Cu") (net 11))
 (segment (start 142.24 55.88) (end 134.08 55.88) (width 0.25) (layer "F.Cu") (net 13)))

